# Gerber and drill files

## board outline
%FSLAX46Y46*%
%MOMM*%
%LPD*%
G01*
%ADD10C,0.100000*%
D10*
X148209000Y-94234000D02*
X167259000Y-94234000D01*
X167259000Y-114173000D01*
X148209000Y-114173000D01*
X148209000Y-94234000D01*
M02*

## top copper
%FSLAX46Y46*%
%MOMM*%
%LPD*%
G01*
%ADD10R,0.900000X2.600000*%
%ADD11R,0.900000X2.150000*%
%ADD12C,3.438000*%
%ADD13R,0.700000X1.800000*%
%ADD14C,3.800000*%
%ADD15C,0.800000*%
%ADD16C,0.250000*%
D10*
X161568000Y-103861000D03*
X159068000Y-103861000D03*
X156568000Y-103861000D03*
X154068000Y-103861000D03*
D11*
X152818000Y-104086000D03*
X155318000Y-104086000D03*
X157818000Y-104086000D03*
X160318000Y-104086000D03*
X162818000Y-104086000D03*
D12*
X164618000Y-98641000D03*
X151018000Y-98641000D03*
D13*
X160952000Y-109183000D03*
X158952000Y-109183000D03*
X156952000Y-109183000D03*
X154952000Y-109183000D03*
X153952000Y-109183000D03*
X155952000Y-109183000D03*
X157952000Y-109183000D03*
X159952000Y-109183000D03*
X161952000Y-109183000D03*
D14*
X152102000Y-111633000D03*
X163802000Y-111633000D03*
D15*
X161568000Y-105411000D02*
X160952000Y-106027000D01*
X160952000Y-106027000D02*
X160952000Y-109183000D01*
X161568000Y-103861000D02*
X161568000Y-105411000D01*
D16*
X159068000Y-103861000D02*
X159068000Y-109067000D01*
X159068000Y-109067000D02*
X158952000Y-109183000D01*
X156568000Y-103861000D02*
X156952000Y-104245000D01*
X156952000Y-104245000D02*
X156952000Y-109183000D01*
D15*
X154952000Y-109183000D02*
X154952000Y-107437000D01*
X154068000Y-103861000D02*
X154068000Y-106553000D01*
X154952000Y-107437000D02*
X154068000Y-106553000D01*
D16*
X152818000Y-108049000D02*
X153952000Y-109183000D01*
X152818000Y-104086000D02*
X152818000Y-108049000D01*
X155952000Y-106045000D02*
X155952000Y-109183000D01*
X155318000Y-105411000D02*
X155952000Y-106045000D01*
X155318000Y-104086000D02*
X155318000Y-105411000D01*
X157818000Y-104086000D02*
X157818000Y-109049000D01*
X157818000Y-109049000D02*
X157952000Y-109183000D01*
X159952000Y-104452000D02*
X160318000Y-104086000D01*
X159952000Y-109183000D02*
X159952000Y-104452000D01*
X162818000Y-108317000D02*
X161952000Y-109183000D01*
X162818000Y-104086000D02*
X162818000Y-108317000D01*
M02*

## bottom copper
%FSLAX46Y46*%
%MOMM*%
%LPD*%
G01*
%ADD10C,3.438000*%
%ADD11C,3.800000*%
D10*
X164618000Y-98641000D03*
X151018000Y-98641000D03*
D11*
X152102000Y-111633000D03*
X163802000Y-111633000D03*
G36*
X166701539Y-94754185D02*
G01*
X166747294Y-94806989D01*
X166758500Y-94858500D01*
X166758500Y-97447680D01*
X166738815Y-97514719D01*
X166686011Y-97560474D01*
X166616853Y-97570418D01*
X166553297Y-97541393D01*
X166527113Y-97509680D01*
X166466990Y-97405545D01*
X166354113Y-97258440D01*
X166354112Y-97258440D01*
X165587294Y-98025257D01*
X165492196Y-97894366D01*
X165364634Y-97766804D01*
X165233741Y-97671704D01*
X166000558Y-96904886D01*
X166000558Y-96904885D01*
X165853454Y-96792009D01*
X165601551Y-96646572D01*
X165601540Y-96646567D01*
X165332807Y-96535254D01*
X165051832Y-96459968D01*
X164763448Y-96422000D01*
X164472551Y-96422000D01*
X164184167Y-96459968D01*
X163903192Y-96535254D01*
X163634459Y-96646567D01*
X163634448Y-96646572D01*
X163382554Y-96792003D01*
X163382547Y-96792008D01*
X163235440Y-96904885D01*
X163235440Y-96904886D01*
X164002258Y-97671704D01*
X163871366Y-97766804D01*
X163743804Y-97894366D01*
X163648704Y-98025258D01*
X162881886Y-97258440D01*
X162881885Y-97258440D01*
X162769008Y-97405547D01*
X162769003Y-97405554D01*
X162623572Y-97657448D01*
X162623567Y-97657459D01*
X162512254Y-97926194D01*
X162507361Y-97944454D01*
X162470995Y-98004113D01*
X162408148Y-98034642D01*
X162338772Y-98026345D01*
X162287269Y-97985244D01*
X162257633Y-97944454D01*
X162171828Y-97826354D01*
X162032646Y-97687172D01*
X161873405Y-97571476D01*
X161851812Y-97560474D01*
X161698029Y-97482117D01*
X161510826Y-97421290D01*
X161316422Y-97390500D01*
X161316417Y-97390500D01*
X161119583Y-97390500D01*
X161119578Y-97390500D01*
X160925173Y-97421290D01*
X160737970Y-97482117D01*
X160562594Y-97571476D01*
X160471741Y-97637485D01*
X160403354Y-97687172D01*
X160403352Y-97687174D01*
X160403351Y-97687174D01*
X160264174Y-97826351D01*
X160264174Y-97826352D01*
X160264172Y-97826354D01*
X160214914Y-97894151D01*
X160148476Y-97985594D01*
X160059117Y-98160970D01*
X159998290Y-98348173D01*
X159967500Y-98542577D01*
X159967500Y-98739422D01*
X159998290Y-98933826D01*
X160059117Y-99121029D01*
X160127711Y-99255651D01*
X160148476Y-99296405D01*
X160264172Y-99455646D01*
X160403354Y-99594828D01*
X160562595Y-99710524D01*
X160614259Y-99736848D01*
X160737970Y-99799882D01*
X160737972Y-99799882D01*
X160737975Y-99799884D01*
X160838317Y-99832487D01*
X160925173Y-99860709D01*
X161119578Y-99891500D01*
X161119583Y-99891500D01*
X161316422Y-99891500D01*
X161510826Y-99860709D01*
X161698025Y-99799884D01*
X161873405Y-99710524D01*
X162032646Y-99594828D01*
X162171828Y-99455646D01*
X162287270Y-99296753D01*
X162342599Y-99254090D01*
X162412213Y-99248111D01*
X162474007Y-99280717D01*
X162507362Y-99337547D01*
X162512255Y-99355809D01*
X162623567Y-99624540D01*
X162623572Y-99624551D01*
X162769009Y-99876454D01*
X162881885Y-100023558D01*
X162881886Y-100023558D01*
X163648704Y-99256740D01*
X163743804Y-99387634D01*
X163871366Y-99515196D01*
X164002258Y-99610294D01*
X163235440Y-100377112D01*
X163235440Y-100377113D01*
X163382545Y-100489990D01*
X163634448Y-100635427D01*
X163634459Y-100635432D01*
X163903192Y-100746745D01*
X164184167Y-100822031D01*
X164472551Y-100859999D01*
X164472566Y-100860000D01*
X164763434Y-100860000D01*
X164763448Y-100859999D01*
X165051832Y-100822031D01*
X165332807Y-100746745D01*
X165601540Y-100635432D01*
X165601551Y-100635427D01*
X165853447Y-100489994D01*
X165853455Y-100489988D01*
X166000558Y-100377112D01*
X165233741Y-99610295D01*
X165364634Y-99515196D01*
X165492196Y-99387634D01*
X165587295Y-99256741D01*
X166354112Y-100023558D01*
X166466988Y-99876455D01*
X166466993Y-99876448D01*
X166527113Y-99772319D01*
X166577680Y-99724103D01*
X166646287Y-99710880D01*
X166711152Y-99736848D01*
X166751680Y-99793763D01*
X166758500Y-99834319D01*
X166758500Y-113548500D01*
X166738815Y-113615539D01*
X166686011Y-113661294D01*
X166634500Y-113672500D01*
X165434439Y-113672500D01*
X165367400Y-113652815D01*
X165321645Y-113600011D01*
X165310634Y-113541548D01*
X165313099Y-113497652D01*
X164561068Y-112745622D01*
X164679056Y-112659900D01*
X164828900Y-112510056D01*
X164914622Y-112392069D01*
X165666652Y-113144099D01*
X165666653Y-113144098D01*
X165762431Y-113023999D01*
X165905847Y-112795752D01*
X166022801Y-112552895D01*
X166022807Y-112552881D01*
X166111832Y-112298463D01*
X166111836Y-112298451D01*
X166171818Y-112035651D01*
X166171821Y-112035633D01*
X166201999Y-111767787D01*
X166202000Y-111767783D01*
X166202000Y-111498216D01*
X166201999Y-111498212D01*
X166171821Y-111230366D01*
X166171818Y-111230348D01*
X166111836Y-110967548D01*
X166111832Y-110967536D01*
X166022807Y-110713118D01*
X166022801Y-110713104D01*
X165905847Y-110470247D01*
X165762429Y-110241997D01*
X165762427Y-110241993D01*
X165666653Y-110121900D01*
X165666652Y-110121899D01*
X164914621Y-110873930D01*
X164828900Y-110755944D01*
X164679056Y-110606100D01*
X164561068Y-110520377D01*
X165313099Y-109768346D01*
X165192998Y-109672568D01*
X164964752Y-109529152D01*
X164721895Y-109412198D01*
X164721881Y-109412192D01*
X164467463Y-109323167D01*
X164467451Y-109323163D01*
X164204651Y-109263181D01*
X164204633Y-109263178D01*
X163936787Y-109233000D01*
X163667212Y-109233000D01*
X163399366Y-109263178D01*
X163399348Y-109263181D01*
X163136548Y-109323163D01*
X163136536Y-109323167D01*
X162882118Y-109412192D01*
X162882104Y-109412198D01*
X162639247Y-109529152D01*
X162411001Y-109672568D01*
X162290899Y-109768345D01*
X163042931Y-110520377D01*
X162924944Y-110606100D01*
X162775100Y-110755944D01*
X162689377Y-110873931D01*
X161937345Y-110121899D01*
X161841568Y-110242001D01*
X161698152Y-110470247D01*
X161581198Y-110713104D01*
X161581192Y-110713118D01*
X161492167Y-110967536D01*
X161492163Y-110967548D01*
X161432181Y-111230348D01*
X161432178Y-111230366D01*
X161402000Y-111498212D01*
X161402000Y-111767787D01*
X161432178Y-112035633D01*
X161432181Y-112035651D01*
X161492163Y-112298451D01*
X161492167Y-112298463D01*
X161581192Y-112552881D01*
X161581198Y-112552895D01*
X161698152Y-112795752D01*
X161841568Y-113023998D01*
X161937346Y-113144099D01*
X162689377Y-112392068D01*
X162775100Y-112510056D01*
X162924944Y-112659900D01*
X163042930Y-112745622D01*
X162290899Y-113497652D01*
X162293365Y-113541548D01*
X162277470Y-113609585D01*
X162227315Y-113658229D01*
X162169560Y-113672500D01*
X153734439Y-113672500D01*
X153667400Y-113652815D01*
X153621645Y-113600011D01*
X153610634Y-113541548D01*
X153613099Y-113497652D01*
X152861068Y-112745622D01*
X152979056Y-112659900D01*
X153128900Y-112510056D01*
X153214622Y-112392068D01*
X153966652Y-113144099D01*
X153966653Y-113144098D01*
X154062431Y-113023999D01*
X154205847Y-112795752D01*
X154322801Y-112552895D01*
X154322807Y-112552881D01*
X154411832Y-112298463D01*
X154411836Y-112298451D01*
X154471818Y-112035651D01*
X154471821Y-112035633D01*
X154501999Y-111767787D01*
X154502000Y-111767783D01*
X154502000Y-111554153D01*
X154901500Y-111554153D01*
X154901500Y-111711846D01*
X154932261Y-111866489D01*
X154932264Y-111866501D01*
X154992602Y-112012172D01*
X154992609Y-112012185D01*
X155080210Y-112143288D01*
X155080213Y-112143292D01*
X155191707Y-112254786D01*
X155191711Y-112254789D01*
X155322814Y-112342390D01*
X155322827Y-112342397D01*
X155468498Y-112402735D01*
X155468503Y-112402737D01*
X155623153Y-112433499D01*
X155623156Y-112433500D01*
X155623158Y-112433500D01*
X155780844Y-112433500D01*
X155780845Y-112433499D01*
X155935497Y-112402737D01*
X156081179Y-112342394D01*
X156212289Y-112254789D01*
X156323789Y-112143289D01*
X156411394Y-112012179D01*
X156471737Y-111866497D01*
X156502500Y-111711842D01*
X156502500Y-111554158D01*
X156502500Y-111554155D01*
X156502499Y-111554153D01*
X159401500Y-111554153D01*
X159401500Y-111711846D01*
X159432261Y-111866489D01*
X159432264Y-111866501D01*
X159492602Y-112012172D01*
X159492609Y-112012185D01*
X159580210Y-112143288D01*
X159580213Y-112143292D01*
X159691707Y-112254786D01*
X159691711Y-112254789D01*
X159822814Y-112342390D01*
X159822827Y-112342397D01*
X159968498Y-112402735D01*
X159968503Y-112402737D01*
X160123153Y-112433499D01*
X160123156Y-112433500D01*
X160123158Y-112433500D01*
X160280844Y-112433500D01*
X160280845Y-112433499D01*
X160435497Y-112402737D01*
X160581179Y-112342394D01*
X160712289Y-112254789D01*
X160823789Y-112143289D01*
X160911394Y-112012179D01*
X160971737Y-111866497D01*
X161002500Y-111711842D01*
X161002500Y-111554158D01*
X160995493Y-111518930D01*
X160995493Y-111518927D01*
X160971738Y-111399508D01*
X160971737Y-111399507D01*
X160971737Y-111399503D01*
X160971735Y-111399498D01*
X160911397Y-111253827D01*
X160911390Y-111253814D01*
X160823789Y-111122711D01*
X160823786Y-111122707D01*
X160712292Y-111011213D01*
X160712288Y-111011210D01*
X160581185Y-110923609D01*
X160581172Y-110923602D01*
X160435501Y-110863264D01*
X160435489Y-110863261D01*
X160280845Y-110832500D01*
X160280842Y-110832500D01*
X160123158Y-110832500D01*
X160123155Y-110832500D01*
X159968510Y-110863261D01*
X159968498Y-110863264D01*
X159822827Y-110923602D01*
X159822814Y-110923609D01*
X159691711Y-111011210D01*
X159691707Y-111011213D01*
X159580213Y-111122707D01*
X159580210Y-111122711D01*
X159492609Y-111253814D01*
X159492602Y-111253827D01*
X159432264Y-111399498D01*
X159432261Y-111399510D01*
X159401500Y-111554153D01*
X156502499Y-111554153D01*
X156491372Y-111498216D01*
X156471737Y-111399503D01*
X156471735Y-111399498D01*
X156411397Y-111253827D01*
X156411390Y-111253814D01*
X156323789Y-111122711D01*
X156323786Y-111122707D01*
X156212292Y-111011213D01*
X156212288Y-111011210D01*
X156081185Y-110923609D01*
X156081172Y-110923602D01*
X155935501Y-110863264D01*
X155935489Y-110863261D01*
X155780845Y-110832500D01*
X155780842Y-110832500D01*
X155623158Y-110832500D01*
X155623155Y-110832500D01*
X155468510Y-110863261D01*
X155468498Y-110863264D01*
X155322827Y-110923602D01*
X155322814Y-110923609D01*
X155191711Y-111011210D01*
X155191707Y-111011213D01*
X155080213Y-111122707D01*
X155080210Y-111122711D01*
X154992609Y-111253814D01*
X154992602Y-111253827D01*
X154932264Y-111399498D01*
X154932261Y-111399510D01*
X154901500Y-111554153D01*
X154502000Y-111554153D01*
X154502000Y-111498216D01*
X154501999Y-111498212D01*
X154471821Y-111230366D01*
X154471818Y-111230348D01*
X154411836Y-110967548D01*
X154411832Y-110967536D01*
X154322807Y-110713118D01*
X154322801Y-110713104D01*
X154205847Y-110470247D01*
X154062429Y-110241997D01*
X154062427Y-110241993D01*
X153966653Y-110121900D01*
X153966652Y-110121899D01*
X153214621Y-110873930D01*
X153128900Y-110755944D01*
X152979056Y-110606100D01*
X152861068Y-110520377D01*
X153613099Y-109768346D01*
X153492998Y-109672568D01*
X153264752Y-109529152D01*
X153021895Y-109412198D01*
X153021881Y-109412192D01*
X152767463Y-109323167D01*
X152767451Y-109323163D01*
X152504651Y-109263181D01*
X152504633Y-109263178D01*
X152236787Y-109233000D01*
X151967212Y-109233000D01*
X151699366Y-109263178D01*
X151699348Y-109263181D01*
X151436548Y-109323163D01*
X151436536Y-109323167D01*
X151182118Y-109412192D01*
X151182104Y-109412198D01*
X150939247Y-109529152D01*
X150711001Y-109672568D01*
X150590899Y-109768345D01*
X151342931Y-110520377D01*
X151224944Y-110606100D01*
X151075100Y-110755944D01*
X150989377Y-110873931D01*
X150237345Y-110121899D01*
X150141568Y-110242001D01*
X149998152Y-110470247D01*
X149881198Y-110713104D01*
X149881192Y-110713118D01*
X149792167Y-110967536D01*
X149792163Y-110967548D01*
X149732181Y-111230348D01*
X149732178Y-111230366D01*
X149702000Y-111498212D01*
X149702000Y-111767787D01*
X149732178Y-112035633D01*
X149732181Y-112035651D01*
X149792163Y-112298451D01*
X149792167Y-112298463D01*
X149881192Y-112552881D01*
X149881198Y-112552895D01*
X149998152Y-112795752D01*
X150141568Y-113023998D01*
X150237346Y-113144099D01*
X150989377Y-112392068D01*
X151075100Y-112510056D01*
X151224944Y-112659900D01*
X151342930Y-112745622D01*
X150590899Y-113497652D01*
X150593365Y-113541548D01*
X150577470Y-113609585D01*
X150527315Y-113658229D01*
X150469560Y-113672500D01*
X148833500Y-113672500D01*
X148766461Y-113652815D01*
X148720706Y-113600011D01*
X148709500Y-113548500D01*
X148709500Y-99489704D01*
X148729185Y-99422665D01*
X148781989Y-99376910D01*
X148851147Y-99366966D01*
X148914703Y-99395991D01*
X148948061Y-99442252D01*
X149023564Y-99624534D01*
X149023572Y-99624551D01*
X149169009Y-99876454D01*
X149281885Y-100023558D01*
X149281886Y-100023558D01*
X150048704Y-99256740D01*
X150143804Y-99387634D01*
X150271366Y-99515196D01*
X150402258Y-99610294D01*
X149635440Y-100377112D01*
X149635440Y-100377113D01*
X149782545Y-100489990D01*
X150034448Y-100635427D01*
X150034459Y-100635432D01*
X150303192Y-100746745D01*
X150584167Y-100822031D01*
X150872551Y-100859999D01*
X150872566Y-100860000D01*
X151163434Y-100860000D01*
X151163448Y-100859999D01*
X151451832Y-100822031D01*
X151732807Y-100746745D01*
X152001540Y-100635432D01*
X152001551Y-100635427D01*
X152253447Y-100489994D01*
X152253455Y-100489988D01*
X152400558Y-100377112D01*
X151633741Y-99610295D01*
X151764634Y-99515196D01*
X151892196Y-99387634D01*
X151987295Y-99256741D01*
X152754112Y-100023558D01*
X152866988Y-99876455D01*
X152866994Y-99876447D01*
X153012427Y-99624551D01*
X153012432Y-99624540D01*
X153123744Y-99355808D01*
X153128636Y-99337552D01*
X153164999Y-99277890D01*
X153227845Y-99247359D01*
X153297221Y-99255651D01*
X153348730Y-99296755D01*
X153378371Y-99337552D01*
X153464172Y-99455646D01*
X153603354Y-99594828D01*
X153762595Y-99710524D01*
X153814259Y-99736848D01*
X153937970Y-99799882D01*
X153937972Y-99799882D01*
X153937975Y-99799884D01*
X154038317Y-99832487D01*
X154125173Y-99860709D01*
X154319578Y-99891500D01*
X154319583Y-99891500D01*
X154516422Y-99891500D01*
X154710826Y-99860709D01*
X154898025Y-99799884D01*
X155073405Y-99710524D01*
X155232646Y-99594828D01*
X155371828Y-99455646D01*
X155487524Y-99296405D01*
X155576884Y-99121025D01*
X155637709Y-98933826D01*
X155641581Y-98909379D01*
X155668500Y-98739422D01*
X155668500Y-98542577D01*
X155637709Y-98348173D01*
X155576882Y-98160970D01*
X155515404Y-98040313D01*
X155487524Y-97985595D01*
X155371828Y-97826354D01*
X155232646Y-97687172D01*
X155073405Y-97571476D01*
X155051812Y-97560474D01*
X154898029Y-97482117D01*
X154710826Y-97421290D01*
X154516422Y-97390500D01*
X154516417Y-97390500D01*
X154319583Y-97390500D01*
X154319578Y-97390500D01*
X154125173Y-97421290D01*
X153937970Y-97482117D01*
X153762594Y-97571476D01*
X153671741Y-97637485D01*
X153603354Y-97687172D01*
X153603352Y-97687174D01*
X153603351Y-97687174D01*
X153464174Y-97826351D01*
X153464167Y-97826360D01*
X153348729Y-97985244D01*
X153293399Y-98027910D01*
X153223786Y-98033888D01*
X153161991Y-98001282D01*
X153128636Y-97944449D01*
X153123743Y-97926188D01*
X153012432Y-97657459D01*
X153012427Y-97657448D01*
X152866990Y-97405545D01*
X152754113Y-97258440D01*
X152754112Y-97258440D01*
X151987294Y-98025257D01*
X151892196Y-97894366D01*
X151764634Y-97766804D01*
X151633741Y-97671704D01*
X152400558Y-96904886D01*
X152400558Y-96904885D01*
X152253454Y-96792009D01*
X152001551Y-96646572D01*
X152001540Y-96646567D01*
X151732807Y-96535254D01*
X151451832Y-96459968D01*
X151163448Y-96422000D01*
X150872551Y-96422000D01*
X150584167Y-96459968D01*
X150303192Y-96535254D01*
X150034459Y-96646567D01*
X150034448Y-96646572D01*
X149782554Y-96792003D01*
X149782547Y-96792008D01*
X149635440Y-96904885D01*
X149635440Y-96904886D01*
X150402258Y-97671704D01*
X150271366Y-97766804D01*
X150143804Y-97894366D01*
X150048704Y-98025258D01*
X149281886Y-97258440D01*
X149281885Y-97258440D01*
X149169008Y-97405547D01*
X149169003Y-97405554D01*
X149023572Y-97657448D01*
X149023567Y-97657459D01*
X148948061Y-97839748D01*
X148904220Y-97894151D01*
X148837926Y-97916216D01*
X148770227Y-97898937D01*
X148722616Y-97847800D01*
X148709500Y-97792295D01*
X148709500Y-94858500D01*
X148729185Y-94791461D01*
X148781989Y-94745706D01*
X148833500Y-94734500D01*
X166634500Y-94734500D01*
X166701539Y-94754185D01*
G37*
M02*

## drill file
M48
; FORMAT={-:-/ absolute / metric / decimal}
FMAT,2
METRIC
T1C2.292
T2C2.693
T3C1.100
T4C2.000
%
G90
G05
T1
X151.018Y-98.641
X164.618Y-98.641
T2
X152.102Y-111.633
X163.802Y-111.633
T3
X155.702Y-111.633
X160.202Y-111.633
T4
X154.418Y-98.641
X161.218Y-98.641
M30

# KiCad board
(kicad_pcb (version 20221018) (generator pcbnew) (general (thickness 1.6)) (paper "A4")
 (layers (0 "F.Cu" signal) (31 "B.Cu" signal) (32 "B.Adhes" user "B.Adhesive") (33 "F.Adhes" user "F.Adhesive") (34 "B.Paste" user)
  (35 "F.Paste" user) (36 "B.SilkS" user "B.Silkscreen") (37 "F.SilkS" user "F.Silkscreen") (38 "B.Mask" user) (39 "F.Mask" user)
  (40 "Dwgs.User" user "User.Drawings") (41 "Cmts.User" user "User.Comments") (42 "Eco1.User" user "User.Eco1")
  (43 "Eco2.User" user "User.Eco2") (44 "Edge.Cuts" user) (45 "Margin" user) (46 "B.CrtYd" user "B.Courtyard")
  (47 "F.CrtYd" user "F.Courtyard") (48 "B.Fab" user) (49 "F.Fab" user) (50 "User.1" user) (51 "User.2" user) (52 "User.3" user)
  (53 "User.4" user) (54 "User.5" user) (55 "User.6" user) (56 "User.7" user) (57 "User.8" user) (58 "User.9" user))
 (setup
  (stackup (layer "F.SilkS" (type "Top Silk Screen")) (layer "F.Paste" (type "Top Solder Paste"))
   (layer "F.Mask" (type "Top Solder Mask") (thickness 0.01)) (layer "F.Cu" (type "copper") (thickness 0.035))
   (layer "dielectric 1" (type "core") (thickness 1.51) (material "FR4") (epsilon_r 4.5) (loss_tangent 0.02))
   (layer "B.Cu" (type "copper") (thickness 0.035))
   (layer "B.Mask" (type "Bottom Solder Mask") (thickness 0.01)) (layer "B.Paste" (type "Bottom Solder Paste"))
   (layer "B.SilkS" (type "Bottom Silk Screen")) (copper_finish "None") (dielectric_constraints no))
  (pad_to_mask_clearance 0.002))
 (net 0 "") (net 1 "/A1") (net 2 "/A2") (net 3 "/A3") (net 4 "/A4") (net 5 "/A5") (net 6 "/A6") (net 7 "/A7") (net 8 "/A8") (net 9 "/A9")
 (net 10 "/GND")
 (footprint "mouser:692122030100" (layer "F.Cu") (at 157.818 98.641 180)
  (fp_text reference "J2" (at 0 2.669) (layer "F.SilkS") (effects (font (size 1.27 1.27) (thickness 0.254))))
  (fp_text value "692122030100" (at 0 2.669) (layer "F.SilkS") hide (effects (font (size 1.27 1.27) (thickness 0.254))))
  (pad "" np_thru_hole circle (at -3.4 0 180) (size 0.001 0.001) (drill 2) (layers "*.Cu" "*.Mask"))
  (pad "" np_thru_hole circle (at 3.4 0 180) (size 0.001 0.001) (drill 2) (layers "*.Cu" "*.Mask"))
  (pad "1" smd rect (at -3.75 -5.22 180) (size 0.9 2.6) (layers "F.Cu" "F.Paste" "F.Mask") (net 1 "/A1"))
  (pad "2" smd rect (at -1.25 -5.22 180) (size 0.9 2.6) (layers "F.Cu" "F.Paste" "F.Mask") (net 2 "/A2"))
  (pad "3" smd rect (at 1.25 -5.22 180) (size 0.9 2.6) (layers "F.Cu" "F.Paste" "F.Mask") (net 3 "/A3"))
  (pad "4" smd rect (at 3.75 -5.22 180) (size 0.9 2.6) (layers "F.Cu" "F.Paste" "F.Mask") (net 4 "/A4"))
  (pad "5" smd rect (at 5 -5.445 180) (size 0.9 2.15) (layers "F.Cu" "F.Paste" "F.Mask") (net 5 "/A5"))
  (pad "6" smd rect (at 2.5 -5.445 180) (size 0.9 2.15) (layers "F.Cu" "F.Paste" "F.Mask") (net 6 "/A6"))
  (pad "7" smd rect (at 0 -5.445 180) (size 0.9 2.15) (layers "F.Cu" "F.Paste" "F.Mask") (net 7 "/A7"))
  (pad "8" smd rect (at -2.5 -5.445 180) (size 0.9 2.15) (layers "F.Cu" "F.Paste" "F.Mask") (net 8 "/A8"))
  (pad "9" smd rect (at -5 -5.445 180) (size 0.9 2.15) (layers "F.Cu" "F.Paste" "F.Mask") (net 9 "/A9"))
  (pad "MH1" thru_hole circle (at -6.8 0 180) (size 3.438 3.438) (drill 2.2922) (layers "*.Cu" "*.Mask") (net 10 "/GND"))
  (pad "MH2" thru_hole circle (at 6.8 0 180) (size 3.438 3.438) (drill 2.2922) (layers "*.Cu" "*.Mask") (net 10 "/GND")))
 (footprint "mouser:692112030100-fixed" (layer "F.Cu") (at 157.952 111.458)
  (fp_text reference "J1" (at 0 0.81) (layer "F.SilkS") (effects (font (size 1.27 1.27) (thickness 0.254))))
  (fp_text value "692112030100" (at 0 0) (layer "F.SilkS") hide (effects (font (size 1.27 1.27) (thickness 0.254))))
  (pad "" np_thru_hole circle (at -2.25 0.175) (size 0.001 0.001) (drill 1.1) (layers "*.Cu" "*.Mask"))
  (pad "" np_thru_hole circle (at 2.25 0.175) (size 0.001 0.001) (drill 1.1) (layers "*.Cu" "*.Mask"))
  (pad "1" smd rect (at 3 -2.275) (size 0.7 1.8) (layers "F.Cu" "F.Paste" "F.Mask") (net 1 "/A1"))
  (pad "2" smd rect (at 1 -2.275) (size 0.7 1.8) (layers "F.Cu" "F.Paste" "F.Mask") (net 2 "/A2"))
  (pad "3" smd rect (at -1 -2.275) (size 0.7 1.8) (layers "F.Cu" "F.Paste" "F.Mask") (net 3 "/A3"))
  (pad "4" smd rect (at -3 -2.275) (size 0.7 1.8) (layers "F.Cu" "F.Paste" "F.Mask") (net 4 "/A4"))
  (pad "5" smd rect (at -4 -2.275) (size 0.7 1.8) (layers "F.Cu" "F.Paste" "F.Mask") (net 5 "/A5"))
  (pad "6" smd rect (at -2 -2.275) (size 0.7 1.8) (layers "F.Cu" "F.Paste" "F.Mask") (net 6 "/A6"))
  (pad "7" smd rect (at 0 -2.275) (size 0.7 1.8) (layers "F.Cu" "F.Paste" "F.Mask") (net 7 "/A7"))
  (pad "8" smd rect (at 2 -2.275) (size 0.7 1.8) (layers "F.Cu" "F.Paste" "F.Mask") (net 8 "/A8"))
  (pad "9" smd rect (at 4 -2.275) (size 0.7 1.8) (layers "F.Cu" "F.Paste" "F.Mask") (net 9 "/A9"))
  (pad "10" thru_hole circle (at -5.85 0.175) (size 3.8 3.8) (drill 2.6926) (layers "*.Cu" "*.Mask") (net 10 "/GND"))
  (pad "11" thru_hole circle (at 5.85 0.175) (size 3.8 3.8) (drill 2.6926) (layers "*.Cu" "*.Mask") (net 10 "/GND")))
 (gr_rect (start 148.209 94.234) (end 167.259 114.173) (stroke (width 0.1) (type default)) (fill none) (layer "Edge.Cuts"))
 (segment (start 161.568 105.411) (end 160.952 106.027) (width 0.8) (layer "F.Cu") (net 1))
 (segment (start 160.952 106.027) (end 160.952 109.183) (width 0.8) (layer "F.Cu") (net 1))
 (segment (start 161.568 103.861) (end 161.568 105.411) (width 0.8) (layer "F.Cu") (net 1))
 (segment (start 159.068 103.861) (end 159.068 109.067) (width 0.25) (layer "F.Cu") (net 2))
 (segment (start 159.068 109.067) (end 158.952 109.183) (width 0.25) (layer "F.Cu") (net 2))
 (segment (start 156.568 103.861) (end 156.952 104.245) (width 0.25) (layer "F.Cu") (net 3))
 (segment (start 156.952 104.245) (end 156.952 109.183) (width 0.25) (layer "F.Cu") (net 3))
 (segment (start 154.952 109.183) (end 154.952 107.437) (width 0.8) (layer "F.Cu") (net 4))
 (segment (start 154.068 103.861) (end 154.068 106.553) (width 0.8) (layer "F.Cu") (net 4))
 (segment (start 154.952 107.437) (end 154.068 106.553) (width 0.8) (layer "F.Cu") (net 4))
 (segment (start 152.818 108.049) (end 153.952 109.183) (width 0.25) (layer "F.Cu") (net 5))
 (segment (start 152.818 104.086) (end 152.818 108.049) (width 0.25) (layer "F.Cu") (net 5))
 (segment (start 155.952 106.045) (end 155.952 109.183) (width 0.25) (layer "F.Cu") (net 6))
 (segment (start 155.318 105.411) (end 155.952 106.045) (width 0.25) (layer "F.Cu") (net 6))
 (segment (start 155.318 104.086) (end 155.318 105.411) (width 0.25) (layer "F.Cu") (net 6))
 (segment (start 157.818 104.086) (end 157.818 109.049) (width 0.25) (layer "F.Cu") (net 7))
 (segment (start 157.818 109.049) (end 157.952 109.183) (width 0.25) (layer "F.Cu") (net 7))
 (segment (start 159.952 104.452) (end 160.318 104.086) (width 0.25) (layer "F.Cu") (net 8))
 (segment (start 159.952 109.183) (end 159.952 104.452) (width 0.25) (layer "F.Cu") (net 8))
 (segment (start 162.818 108.317) (end 161.952 109.183) (width 0.25) (layer "F.Cu") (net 9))
 (segment (start 162.818 104.086) (end 162.818 108.317) (width 0.25) (layer "F.Cu") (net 9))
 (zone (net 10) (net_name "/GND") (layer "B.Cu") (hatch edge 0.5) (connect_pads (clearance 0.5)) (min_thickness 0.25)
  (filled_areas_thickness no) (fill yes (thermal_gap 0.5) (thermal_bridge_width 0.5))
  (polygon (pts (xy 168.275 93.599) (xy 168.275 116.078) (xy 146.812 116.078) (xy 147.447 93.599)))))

